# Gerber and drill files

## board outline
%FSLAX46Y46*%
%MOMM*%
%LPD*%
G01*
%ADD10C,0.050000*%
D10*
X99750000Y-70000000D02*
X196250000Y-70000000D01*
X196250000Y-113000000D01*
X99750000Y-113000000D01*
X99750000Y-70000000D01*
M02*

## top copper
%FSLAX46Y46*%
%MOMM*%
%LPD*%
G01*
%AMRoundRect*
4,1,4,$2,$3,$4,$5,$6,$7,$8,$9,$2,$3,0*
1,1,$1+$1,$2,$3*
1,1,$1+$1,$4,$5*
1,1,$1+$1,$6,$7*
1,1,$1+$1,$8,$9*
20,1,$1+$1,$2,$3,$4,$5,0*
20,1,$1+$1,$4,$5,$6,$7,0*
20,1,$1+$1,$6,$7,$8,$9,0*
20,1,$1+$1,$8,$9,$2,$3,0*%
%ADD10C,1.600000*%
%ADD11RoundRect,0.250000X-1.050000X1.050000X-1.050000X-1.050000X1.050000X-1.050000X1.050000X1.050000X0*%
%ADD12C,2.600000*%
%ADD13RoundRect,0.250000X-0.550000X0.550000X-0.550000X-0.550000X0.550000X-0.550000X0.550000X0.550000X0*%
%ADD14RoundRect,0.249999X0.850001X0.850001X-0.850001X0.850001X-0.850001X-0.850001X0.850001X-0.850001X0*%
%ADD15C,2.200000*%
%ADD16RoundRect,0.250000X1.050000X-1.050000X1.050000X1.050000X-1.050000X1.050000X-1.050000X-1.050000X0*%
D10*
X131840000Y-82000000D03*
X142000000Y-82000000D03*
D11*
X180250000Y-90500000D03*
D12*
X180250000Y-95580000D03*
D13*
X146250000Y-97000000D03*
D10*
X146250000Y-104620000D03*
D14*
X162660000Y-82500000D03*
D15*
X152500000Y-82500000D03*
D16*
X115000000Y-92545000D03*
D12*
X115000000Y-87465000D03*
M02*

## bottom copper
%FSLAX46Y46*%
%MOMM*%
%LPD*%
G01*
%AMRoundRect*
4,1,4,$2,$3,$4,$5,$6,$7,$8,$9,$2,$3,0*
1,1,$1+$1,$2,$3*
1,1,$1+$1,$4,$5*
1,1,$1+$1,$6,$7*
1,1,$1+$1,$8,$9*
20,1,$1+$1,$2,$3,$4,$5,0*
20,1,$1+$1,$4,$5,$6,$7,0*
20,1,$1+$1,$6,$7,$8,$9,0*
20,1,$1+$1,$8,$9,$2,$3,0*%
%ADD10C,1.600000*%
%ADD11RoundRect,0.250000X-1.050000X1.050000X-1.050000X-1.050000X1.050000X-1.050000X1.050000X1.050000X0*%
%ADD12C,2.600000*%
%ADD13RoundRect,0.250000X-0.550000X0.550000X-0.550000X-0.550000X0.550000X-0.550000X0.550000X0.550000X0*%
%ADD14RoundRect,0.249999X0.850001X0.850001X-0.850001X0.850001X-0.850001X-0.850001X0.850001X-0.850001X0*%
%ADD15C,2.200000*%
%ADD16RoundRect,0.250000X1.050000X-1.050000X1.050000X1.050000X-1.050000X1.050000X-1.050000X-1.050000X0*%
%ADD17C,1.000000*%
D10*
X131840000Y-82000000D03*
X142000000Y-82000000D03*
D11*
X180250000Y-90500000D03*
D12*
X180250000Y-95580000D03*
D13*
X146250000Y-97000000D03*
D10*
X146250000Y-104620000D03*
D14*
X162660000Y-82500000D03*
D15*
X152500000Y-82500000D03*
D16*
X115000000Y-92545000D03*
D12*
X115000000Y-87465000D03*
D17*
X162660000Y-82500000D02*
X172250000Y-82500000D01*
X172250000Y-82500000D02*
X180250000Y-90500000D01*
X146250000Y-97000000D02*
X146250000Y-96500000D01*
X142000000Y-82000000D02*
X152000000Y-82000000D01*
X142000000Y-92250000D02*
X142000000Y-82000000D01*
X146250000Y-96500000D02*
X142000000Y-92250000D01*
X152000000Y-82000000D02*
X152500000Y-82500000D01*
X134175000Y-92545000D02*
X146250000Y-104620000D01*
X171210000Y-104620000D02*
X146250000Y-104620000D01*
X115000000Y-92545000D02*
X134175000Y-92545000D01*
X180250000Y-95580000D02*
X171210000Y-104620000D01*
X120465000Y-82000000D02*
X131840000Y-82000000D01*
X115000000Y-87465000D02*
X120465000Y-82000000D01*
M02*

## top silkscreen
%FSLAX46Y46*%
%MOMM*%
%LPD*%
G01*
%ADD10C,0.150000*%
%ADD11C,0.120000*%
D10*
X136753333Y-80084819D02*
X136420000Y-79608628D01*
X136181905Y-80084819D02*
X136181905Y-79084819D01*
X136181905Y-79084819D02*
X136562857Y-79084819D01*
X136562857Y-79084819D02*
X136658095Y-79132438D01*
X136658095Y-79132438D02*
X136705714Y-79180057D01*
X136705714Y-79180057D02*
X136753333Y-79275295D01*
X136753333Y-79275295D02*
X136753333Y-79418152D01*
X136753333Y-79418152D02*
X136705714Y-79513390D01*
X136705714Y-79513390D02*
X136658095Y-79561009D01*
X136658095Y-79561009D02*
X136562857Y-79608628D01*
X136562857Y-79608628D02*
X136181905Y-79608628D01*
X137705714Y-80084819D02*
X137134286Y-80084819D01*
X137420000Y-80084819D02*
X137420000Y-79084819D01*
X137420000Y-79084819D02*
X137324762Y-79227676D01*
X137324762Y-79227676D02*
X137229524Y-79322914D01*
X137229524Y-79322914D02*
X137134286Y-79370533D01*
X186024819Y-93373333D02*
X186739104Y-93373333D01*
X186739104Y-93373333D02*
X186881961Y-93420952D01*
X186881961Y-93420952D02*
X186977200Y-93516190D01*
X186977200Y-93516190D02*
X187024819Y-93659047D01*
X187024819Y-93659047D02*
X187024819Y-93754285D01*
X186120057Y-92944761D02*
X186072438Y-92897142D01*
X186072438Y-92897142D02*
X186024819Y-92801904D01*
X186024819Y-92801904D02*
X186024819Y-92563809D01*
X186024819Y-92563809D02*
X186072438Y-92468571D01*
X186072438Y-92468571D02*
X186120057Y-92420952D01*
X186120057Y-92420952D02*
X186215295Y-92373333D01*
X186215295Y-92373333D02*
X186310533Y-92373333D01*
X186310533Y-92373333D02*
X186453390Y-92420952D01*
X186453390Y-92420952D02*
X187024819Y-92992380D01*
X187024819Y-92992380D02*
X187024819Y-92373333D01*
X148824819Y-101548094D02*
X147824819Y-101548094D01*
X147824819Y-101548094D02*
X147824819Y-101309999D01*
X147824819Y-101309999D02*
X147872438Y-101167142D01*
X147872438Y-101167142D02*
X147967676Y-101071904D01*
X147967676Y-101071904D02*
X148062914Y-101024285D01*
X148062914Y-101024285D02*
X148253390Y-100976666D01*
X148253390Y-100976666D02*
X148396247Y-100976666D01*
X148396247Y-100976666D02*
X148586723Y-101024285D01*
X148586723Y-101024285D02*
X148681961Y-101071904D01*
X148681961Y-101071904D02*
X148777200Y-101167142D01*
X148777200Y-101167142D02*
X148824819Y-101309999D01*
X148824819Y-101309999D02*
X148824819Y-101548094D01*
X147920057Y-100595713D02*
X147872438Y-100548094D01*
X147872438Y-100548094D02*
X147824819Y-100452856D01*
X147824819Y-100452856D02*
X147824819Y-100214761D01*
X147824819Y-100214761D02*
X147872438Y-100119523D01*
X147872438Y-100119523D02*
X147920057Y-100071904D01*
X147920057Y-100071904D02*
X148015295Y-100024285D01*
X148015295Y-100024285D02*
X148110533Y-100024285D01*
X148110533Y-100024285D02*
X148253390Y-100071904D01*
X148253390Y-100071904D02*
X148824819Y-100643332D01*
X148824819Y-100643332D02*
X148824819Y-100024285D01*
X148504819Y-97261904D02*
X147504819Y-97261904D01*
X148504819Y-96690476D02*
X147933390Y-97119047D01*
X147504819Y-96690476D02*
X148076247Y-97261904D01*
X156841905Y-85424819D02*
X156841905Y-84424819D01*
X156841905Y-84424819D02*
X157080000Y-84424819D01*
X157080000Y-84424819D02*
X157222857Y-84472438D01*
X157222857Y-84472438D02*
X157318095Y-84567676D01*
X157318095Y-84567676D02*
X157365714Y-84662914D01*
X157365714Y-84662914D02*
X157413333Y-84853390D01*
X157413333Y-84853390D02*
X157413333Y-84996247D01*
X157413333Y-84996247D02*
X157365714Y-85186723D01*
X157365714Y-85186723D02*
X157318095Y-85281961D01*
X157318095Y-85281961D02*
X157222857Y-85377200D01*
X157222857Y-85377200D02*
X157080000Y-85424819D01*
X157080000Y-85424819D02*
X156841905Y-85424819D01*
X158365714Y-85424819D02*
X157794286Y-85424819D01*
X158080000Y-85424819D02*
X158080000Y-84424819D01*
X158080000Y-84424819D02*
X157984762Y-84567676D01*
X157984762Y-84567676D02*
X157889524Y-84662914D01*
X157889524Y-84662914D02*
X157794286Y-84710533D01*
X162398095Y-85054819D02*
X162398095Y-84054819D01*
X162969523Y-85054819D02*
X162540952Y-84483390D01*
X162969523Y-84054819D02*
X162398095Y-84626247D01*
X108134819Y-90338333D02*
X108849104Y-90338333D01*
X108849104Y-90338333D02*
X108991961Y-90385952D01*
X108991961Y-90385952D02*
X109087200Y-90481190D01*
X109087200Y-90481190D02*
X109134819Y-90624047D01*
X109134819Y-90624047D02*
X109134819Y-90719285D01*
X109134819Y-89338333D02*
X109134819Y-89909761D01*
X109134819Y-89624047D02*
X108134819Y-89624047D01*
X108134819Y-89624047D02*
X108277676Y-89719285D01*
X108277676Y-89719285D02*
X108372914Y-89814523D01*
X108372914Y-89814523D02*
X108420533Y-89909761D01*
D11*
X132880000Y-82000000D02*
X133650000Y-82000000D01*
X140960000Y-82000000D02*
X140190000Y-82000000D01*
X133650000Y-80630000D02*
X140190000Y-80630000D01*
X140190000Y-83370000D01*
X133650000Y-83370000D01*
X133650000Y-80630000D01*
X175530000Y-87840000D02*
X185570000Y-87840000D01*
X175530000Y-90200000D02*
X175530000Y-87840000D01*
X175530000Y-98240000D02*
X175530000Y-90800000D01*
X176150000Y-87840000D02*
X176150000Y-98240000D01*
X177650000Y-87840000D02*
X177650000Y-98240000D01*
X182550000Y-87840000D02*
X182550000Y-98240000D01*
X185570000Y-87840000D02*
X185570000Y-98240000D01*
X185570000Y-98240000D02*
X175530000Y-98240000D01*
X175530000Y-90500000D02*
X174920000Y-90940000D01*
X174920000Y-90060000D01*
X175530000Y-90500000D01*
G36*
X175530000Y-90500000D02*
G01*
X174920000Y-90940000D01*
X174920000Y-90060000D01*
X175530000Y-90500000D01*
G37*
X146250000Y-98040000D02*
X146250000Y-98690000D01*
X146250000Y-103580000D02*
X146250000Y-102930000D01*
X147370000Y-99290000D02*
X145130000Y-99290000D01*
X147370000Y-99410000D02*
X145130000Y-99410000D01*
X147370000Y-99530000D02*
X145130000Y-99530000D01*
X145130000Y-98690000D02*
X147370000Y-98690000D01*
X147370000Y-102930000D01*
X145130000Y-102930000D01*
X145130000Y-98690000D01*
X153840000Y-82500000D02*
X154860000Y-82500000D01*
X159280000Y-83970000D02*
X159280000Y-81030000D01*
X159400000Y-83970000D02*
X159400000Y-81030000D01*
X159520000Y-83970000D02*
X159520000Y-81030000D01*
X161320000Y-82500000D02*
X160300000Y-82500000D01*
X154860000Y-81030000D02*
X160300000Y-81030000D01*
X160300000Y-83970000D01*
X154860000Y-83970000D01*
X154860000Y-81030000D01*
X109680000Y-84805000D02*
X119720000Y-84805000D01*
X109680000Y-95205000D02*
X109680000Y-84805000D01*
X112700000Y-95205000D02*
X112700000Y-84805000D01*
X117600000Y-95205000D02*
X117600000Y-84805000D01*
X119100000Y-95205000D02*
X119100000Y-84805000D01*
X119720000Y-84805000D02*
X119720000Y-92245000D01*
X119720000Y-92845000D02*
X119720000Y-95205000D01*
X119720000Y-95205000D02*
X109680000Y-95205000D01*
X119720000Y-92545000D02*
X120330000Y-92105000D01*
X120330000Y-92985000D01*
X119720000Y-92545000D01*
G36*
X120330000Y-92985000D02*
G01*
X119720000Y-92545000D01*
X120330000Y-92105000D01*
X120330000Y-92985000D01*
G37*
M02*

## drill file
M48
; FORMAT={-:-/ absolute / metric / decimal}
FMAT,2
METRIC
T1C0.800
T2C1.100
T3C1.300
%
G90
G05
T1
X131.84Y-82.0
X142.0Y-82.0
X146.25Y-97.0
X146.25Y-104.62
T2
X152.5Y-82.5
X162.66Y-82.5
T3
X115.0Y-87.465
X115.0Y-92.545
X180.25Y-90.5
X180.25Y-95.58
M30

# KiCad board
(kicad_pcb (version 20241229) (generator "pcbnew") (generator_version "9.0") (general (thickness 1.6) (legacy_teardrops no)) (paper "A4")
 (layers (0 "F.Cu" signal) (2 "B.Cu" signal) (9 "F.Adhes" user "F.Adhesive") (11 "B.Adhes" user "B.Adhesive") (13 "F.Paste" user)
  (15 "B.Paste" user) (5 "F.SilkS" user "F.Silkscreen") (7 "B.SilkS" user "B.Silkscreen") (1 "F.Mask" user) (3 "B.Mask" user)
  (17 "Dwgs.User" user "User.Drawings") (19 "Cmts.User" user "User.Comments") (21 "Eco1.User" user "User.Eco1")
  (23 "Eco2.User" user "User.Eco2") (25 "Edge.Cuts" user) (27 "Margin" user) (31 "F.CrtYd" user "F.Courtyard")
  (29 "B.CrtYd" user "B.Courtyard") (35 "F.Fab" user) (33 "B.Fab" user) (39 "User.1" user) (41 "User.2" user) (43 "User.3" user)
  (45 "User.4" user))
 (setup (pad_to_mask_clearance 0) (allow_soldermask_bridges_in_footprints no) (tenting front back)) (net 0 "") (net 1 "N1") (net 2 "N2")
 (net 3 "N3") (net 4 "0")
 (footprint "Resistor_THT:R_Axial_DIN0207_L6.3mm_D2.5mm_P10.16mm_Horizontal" (layer "F.Cu") (at 131.84 82)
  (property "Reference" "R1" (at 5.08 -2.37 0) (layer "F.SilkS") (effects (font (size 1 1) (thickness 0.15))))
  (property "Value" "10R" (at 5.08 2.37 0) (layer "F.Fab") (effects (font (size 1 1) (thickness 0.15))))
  (fp_line (start 1.04 0) (end 1.81 0) (stroke (width 0.12) (type solid)) (layer "F.SilkS"))
  (fp_line (start 9.12 0) (end 8.35 0) (stroke (width 0.12) (type solid)) (layer "F.SilkS"))
  (fp_rect (start 1.81 -1.37) (end 8.35 1.37) (stroke (width 0.12) (type solid)) (fill no) (layer "F.SilkS"))
  (pad "1" thru_hole circle (at 0 0) (size 1.6 1.6) (drill 0.8) (layers "*.Cu" "*.Mask") (remove_unused_layers no) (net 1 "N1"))
  (pad "2" thru_hole circle (at 10.16 0) (size 1.6 1.6) (drill 0.8) (layers "*.Cu" "*.Mask") (remove_unused_layers no) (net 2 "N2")))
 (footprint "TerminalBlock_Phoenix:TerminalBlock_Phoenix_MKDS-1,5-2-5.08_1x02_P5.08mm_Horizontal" (layer "F.Cu") (at 180.25 90.5 -90)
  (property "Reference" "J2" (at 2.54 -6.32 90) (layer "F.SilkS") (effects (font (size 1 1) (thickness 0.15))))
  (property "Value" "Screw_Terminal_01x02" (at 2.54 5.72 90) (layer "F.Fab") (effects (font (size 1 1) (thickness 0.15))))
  (fp_line (start -2.66 4.72) (end -2.66 -5.32) (stroke (width 0.12) (type solid)) (layer "F.SilkS"))
  (fp_line (start -0.3 4.72) (end -2.66 4.72) (stroke (width 0.12) (type solid)) (layer "F.SilkS"))
  (fp_line (start 7.74 4.72) (end 0.3 4.72) (stroke (width 0.12) (type solid)) (layer "F.SilkS"))
  (fp_line (start -2.66 4.1) (end 7.74 4.1) (stroke (width 0.12) (type solid)) (layer "F.SilkS"))
  (fp_line (start -2.66 2.6) (end 7.74 2.6) (stroke (width 0.12) (type solid)) (layer "F.SilkS"))
  (fp_line (start -2.66 -2.3) (end 7.74 -2.3) (stroke (width 0.12) (type solid)) (layer "F.SilkS"))
  (fp_line (start -2.66 -5.32) (end 7.74 -5.32) (stroke (width 0.12) (type solid)) (layer "F.SilkS"))
  (fp_line (start 7.74 -5.32) (end 7.74 4.72) (stroke (width 0.12) (type solid)) (layer "F.SilkS"))
  (fp_poly (pts (xy 0 4.72) (xy 0.44 5.33) (xy -0.44 5.33)) (stroke (width 0.12) (type solid)) (fill yes) (layer "F.SilkS"))
  (pad "1" thru_hole roundrect (at 0 0 270) (size 2.6 2.6) (drill 1.3) (layers "*.Cu" "*.Mask") (remove_unused_layers no)
   (roundrect_rratio 0.096154) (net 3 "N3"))
  (pad "2" thru_hole circle (at 5.08 0 270) (size 2.6 2.6) (drill 1.3) (layers "*.Cu" "*.Mask") (remove_unused_layers no) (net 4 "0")))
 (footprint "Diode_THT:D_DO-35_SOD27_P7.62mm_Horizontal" (layer "F.Cu") (at 146.25 97 -90)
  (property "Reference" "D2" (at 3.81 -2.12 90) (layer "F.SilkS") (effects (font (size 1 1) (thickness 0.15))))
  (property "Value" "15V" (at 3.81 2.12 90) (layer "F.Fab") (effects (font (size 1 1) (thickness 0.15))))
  (fp_line (start 1.04 0) (end 1.69 0) (stroke (width 0.12) (type solid)) (layer "F.SilkS"))
  (fp_line (start 6.58 0) (end 5.93 0) (stroke (width 0.12) (type solid)) (layer "F.SilkS"))
  (fp_line (start 2.29 -1.12) (end 2.29 1.12) (stroke (width 0.12) (type solid)) (layer "F.SilkS"))
  (fp_line (start 2.41 -1.12) (end 2.41 1.12) (stroke (width 0.12) (type solid)) (layer "F.SilkS"))
  (fp_line (start 2.53 -1.12) (end 2.53 1.12) (stroke (width 0.12) (type solid)) (layer "F.SilkS"))
  (fp_rect (start 1.69 -1.12) (end 5.93 1.12) (stroke (width 0.12) (type solid)) (fill no) (layer "F.SilkS"))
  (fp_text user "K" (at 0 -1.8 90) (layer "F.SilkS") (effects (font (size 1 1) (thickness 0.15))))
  (pad "1" thru_hole roundrect (at 0 0 270) (size 1.6 1.6) (drill 0.8) (layers "*.Cu" "*.Mask") (remove_unused_layers no)
   (roundrect_rratio 0.15625) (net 2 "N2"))
  (pad "2" thru_hole circle (at 7.62 0 270) (size 1.6 1.6) (drill 0.8) (layers "*.Cu" "*.Mask") (remove_unused_layers no) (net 4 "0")))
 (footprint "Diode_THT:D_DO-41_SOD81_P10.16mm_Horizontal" (layer "F.Cu") (at 162.66 82.5 180)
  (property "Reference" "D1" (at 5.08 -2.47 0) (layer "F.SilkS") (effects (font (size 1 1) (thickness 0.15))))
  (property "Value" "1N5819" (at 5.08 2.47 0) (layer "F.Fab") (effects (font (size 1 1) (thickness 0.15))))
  (fp_line (start 8.82 0) (end 7.8 0) (stroke (width 0.12) (type solid)) (layer "F.SilkS"))
  (fp_line (start 3.38 -1.47) (end 3.38 1.47) (stroke (width 0.12) (type solid)) (layer "F.SilkS"))
  (fp_line (start 3.26 -1.47) (end 3.26 1.47) (stroke (width 0.12) (type solid)) (layer "F.SilkS"))
  (fp_line (start 3.14 -1.47) (end 3.14 1.47) (stroke (width 0.12) (type solid)) (layer "F.SilkS"))
  (fp_line (start 1.34 0) (end 2.36 0) (stroke (width 0.12) (type solid)) (layer "F.SilkS"))
  (fp_rect (start 2.36 -1.47) (end 7.8 1.47) (stroke (width 0.12) (type solid)) (fill no) (layer "F.SilkS"))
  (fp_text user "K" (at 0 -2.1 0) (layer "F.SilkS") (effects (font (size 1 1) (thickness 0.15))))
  (pad "1" thru_hole roundrect (at 0 0 180) (size 2.2 2.2) (drill 1.1) (layers "*.Cu" "*.Mask") (remove_unused_layers no)
   (roundrect_rratio 0.113636) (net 3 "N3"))
  (pad "2" thru_hole circle (at 10.16 0 180) (size 2.2 2.2) (drill 1.1) (layers "*.Cu" "*.Mask") (remove_unused_layers no) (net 2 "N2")))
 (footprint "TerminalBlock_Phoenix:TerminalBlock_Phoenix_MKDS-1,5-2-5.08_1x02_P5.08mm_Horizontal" (layer "F.Cu") (at 115 92.545 90)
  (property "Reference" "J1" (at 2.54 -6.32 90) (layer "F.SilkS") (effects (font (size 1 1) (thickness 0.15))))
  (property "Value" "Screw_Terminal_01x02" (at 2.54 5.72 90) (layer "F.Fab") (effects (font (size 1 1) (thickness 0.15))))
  (fp_line (start 7.74 -5.32) (end 7.74 4.72) (stroke (width 0.12) (type solid)) (layer "F.SilkS"))
  (fp_line (start -2.66 -5.32) (end 7.74 -5.32) (stroke (width 0.12) (type solid)) (layer "F.SilkS"))
  (fp_line (start -2.66 -2.3) (end 7.74 -2.3) (stroke (width 0.12) (type solid)) (layer "F.SilkS"))
  (fp_line (start -2.66 2.6) (end 7.74 2.6) (stroke (width 0.12) (type solid)) (layer "F.SilkS"))
  (fp_line (start -2.66 4.1) (end 7.74 4.1) (stroke (width 0.12) (type solid)) (layer "F.SilkS"))
  (fp_line (start 7.74 4.72) (end 0.3 4.72) (stroke (width 0.12) (type solid)) (layer "F.SilkS"))
  (fp_line (start -0.3 4.72) (end -2.66 4.72) (stroke (width 0.12) (type solid)) (layer "F.SilkS"))
  (fp_line (start -2.66 4.72) (end -2.66 -5.32) (stroke (width 0.12) (type solid)) (layer "F.SilkS"))
  (fp_poly (pts (xy 0 4.72) (xy 0.44 5.33) (xy -0.44 5.33)) (stroke (width 0.12) (type solid)) (fill yes) (layer "F.SilkS"))
  (pad "1" thru_hole roundrect (at 0 0 90) (size 2.6 2.6) (drill 1.3) (layers "*.Cu" "*.Mask") (remove_unused_layers no)
   (roundrect_rratio 0.096154) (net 4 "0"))
  (pad "2" thru_hole circle (at 5.08 0 90) (size 2.6 2.6) (drill 1.3) (layers "*.Cu" "*.Mask") (remove_unused_layers no) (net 1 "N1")))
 (gr_rect (start 99.75 70) (end 196.25 113) (stroke (width 0.05) (type default)) (fill no) (layer "Edge.Cuts"))
 (segment (start 162.66 82.5) (end 172.25 82.5) (width 1) (layer "B.Cu") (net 3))
 (segment (start 172.25 82.5) (end 180.25 90.5) (width 1) (layer "B.Cu") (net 3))
 (segment (start 146.25 97) (end 146.25 96.5) (width 1) (layer "B.Cu") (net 2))
 (segment (start 142 82) (end 152 82) (width 1) (layer "B.Cu") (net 2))
 (segment (start 142 92.25) (end 142 82) (width 1) (layer "B.Cu") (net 2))
 (segment (start 146.25 96.5) (end 142 92.25) (width 1) (layer "B.Cu") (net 2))
 (segment (start 152 82) (end 152.5 82.5) (width 1) (layer "B.Cu") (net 2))
 (segment (start 134.175 92.545) (end 146.25 104.62) (width 1) (layer "B.Cu") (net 4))
 (segment (start 171.21 104.62) (end 146.25 104.62) (width 1) (layer "B.Cu") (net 4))
 (segment (start 115 92.545) (end 134.175 92.545) (width 1) (layer "B.Cu") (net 4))
 (segment (start 180.25 95.58) (end 171.21 104.62) (width 1) (layer "B.Cu") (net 4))
 (segment (start 120.465 82) (end 131.84 82) (width 1) (layer "B.Cu") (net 1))
 (segment (start 115 87.465) (end 120.465 82) (width 1) (layer "B.Cu") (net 1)))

